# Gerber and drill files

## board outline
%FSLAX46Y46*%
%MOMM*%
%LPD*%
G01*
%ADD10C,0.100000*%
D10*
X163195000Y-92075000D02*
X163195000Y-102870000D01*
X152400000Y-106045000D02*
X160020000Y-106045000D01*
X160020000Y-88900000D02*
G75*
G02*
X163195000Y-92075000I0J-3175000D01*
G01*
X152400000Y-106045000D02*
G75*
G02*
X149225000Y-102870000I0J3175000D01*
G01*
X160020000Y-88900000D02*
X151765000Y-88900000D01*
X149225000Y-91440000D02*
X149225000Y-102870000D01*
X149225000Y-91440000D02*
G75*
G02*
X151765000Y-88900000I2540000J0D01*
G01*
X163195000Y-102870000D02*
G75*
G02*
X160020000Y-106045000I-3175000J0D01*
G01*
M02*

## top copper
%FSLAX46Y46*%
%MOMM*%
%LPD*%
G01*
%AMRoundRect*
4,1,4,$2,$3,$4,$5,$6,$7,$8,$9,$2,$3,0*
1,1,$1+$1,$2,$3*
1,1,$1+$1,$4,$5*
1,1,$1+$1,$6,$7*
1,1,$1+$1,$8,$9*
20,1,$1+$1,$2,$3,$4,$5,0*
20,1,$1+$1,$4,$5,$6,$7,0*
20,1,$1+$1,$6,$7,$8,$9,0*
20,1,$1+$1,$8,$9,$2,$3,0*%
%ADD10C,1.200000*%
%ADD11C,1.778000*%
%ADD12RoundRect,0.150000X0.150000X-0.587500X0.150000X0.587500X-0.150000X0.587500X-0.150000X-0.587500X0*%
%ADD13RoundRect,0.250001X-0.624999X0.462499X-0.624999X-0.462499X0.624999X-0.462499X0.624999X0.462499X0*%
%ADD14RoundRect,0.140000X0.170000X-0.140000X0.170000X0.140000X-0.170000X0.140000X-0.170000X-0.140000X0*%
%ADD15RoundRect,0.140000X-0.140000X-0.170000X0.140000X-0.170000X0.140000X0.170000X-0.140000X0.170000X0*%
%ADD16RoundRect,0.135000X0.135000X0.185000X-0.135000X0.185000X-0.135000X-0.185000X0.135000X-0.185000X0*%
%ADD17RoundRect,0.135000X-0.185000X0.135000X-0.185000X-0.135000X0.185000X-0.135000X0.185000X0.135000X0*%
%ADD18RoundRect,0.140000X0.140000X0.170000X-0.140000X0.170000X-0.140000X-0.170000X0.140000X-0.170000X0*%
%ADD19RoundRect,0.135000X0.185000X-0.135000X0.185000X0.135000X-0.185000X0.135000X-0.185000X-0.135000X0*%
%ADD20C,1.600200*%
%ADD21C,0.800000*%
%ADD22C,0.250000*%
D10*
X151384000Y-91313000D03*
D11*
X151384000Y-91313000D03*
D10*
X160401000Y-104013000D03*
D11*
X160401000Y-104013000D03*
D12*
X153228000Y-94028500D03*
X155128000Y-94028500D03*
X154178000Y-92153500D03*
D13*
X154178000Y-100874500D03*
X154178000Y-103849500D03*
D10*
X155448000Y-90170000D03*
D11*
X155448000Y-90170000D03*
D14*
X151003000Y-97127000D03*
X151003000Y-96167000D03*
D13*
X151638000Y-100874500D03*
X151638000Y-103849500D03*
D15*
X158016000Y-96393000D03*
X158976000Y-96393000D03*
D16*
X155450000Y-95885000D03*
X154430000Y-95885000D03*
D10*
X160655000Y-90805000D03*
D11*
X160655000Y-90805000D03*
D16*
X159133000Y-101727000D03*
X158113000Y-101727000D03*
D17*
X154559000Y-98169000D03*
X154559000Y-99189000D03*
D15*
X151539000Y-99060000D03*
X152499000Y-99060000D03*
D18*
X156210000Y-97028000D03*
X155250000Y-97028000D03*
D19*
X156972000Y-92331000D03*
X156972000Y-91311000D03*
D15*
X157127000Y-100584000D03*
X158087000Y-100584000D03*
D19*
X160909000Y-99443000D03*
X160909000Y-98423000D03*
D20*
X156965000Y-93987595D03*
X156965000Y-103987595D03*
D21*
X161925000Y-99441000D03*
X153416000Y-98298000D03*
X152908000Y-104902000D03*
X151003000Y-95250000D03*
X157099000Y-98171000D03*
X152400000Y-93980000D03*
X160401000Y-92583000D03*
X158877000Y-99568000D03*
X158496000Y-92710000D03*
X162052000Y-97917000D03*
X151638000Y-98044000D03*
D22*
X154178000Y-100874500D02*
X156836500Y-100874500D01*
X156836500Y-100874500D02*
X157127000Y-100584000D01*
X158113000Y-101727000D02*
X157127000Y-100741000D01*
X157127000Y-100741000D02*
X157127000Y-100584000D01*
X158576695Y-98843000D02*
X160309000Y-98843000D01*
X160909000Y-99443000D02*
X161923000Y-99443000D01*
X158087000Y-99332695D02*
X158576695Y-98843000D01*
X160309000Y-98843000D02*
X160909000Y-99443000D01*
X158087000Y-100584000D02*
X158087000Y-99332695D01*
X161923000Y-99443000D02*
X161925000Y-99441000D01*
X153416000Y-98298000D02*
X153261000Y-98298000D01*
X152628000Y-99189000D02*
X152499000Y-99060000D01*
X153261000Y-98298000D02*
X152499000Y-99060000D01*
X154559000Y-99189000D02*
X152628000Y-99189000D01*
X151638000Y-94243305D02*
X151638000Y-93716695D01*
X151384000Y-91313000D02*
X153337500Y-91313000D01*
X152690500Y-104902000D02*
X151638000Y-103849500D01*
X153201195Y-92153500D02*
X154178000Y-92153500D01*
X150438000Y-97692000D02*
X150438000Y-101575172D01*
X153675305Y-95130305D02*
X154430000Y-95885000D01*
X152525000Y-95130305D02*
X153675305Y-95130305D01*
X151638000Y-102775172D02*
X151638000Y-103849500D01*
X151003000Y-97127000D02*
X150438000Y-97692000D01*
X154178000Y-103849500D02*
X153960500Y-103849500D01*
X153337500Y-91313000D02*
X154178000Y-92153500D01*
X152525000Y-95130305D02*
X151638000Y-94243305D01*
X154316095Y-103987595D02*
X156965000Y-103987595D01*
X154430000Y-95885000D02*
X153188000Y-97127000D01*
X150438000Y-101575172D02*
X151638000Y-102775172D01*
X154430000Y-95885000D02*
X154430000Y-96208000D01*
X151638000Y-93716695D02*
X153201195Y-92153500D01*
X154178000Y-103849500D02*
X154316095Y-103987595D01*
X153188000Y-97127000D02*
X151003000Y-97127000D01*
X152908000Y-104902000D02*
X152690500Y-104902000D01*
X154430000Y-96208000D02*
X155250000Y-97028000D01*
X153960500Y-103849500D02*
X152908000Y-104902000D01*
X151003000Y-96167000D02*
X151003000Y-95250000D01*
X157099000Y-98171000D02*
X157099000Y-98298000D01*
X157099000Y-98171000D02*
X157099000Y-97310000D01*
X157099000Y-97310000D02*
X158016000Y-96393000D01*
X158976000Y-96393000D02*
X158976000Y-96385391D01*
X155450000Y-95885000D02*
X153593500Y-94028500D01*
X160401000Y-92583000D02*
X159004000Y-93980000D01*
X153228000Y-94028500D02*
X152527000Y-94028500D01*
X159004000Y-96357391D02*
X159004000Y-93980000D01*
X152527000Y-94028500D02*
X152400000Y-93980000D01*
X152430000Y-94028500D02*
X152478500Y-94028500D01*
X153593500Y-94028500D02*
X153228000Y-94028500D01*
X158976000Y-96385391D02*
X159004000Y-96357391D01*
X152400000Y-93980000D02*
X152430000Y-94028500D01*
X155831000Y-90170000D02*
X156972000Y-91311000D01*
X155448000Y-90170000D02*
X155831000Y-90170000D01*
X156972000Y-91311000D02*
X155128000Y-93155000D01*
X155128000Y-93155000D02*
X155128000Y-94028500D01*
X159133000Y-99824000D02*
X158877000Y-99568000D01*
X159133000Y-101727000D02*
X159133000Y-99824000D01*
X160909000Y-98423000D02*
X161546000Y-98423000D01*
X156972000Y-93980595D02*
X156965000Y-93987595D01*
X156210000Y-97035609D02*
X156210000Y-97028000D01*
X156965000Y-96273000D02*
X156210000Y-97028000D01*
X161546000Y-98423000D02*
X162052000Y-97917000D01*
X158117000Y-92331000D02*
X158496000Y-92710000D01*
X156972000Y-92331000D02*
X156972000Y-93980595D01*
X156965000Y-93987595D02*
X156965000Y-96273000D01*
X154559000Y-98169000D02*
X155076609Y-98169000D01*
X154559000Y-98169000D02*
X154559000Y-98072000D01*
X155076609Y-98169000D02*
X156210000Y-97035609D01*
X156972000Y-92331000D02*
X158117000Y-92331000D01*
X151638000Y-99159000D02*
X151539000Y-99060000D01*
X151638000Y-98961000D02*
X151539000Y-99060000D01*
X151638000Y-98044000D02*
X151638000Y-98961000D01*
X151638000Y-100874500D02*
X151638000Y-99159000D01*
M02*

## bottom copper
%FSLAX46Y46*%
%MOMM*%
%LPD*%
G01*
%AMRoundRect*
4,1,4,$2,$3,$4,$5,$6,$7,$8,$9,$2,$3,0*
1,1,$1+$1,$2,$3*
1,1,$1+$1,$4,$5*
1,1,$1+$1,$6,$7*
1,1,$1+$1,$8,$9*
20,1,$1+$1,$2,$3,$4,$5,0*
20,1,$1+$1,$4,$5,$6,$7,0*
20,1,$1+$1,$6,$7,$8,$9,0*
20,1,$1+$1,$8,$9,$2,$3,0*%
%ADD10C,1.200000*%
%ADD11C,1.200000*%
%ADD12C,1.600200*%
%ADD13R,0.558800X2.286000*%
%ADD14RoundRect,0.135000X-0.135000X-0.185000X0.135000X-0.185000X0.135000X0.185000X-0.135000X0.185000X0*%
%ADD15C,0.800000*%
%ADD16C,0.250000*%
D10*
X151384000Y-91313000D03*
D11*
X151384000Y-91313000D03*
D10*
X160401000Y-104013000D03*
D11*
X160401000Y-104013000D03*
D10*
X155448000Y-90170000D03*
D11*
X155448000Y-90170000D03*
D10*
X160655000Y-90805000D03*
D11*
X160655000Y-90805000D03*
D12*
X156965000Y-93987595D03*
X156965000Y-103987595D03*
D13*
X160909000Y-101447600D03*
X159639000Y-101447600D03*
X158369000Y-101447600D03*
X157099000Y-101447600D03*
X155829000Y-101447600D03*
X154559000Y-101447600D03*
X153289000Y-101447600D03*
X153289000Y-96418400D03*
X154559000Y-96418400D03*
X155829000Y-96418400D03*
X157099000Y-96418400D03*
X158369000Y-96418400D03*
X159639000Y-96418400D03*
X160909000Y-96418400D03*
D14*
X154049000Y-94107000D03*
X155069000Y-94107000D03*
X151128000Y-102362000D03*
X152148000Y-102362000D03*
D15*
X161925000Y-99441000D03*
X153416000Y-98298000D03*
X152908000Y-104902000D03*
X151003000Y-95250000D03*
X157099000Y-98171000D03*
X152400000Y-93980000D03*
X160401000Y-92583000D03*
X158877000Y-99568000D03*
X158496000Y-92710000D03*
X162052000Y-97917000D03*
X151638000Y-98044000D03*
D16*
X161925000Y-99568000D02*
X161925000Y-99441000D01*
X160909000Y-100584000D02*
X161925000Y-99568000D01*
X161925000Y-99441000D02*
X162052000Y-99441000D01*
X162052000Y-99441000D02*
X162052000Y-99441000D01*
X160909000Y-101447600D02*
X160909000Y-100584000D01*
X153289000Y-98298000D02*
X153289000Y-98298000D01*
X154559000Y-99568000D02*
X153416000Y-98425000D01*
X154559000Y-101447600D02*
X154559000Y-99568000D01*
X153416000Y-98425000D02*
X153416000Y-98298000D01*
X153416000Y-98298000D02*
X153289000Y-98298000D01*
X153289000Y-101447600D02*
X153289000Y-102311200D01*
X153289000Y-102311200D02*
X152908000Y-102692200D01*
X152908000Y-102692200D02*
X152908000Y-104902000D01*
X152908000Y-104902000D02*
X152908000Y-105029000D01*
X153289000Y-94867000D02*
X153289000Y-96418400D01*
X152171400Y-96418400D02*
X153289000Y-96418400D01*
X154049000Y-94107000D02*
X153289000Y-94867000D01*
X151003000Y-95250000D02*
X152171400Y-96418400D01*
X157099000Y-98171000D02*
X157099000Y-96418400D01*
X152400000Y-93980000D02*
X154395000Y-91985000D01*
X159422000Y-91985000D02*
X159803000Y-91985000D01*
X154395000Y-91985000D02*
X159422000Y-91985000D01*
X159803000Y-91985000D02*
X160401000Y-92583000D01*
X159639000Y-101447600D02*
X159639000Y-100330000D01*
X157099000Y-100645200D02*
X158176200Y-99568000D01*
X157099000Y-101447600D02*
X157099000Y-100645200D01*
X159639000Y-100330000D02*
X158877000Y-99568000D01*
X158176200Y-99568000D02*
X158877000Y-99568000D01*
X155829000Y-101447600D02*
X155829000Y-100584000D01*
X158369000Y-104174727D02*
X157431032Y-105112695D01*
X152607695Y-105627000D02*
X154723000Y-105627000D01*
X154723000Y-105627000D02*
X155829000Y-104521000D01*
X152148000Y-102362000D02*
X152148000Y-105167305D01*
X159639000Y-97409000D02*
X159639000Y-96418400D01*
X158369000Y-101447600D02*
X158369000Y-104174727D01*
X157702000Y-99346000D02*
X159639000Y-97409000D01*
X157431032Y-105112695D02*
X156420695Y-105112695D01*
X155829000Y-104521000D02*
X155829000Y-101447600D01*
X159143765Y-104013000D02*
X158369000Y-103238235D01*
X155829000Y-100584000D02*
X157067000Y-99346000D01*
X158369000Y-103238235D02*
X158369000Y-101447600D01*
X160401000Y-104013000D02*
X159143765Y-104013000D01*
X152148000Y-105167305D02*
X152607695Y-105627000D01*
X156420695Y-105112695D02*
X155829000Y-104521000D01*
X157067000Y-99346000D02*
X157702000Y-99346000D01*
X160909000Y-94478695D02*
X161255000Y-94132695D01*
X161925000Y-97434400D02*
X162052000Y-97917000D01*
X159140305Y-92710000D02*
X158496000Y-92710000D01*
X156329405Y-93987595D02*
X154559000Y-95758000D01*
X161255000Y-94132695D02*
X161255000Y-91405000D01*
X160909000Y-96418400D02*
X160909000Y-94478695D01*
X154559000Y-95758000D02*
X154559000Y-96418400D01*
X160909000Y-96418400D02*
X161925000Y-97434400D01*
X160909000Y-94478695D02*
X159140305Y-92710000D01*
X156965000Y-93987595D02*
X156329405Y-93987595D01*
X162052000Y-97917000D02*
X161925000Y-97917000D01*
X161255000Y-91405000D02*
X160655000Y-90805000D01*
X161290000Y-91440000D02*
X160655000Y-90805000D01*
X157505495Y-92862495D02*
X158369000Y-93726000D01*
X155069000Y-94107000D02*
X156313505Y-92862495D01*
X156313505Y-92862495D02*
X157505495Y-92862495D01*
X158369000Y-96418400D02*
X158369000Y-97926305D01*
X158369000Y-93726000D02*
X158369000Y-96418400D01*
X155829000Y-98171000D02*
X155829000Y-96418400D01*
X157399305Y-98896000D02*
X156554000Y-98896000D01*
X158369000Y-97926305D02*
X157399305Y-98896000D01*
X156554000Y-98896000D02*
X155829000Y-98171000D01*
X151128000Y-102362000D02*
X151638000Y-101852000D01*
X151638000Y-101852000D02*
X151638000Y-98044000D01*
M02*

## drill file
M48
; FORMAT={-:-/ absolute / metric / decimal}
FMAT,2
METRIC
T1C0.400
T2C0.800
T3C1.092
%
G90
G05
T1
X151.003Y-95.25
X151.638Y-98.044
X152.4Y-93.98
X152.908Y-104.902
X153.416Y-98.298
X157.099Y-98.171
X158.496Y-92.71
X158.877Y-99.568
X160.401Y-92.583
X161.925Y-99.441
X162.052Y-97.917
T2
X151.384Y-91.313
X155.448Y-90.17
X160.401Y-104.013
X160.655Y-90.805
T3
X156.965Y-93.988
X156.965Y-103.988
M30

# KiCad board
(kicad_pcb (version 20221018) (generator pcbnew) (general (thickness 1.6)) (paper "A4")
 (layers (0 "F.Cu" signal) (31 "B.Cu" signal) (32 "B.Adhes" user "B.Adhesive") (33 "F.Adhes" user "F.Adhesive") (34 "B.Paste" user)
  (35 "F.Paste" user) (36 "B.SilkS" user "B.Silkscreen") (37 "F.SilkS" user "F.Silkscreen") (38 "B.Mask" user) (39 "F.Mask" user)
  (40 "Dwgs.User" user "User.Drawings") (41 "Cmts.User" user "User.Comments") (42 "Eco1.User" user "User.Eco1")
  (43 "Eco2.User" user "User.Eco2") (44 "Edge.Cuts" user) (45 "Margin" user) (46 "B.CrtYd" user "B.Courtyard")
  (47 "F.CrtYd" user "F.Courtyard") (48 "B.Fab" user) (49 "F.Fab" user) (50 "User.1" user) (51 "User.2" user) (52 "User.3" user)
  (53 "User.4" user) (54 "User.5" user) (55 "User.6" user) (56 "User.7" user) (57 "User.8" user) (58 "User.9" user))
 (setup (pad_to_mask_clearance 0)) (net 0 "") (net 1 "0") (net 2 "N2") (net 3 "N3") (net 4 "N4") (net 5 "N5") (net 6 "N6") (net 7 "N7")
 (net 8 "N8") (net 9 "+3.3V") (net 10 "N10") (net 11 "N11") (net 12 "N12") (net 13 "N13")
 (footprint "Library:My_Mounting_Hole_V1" (layer "F.Cu") (at 151.384 91.313)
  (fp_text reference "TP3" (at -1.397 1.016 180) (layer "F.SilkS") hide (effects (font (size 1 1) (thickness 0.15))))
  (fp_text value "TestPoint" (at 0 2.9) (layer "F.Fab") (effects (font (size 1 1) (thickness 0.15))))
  (pad "1" thru_hole circle (at 0 0) (size 1.2 1.2) (drill 0.8) (layers "*.Cu" "*.Mask") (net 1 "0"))
  (pad "1" connect circle (at 0 0) (size 1.2 1.2) (layers "B.Cu" "B.Mask") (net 1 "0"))
  (pad "1" connect circle (at 0 0) (size 1.778 1.778) (layers "F.Cu" "F.Mask") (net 1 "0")))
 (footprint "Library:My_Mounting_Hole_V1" (layer "F.Cu") (at 160.401 104.013)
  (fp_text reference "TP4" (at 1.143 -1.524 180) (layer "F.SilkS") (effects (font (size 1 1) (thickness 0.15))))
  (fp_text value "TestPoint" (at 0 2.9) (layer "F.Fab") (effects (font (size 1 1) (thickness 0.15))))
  (pad "1" thru_hole circle (at 0 0) (size 1.2 1.2) (drill 0.8) (layers "*.Cu" "*.Mask") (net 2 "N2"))
  (pad "1" connect circle (at 0 0) (size 1.2 1.2) (layers "B.Cu" "B.Mask") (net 2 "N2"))
  (pad "1" connect circle (at 0 0) (size 1.778 1.778) (layers "F.Cu" "F.Mask") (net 2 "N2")))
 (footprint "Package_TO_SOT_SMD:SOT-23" (layer "F.Cu") (at 154.178 93.091 90)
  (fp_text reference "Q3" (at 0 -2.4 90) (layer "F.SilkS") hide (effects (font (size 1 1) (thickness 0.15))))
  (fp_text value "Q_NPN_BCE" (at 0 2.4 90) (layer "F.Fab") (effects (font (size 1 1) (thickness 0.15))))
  (pad "1" smd roundrect (at -0.9375 -0.95 90) (size 1.475 0.6) (layers "F.Cu" "F.Paste" "F.Mask") (roundrect_rratio 0.25) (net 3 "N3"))
  (pad "2" smd roundrect (at -0.9375 0.95 90) (size 1.475 0.6) (layers "F.Cu" "F.Paste" "F.Mask") (roundrect_rratio 0.25) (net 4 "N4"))
  (pad "3" smd roundrect (at 0.9375 0 90) (size 1.475 0.6) (layers "F.Cu" "F.Paste" "F.Mask") (roundrect_rratio 0.25) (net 1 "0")))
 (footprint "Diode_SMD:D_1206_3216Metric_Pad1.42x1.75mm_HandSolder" (layer "F.Cu") (at 154.178 102.362 -90)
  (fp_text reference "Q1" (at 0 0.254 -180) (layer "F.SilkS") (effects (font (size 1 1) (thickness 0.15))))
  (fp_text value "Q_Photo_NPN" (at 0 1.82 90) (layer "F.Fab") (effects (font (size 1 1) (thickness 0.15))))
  (pad "1" smd roundrect (at -1.4875 0 270) (size 1.425 1.75) (layers "F.Cu" "F.Paste" "F.Mask") (roundrect_rratio 0.1754392982)
   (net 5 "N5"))
  (pad "2" smd roundrect (at 1.4875 0 270) (size 1.425 1.75) (layers "F.Cu" "F.Paste" "F.Mask") (roundrect_rratio 0.1754392982) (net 1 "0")))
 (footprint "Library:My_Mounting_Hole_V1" (layer "F.Cu") (at 155.448 90.17)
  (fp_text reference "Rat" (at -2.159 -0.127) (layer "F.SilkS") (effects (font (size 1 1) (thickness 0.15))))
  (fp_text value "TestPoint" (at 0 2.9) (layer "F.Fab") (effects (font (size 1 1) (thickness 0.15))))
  (pad "1" thru_hole circle (at 0 0) (size 1.2 1.2) (drill 0.8) (layers "*.Cu" "*.Mask") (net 4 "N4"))
  (pad "1" connect circle (at 0 0) (size 1.2 1.2) (layers "B.Cu" "B.Mask") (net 4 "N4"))
  (pad "1" connect circle (at 0 0) (size 1.778 1.778) (layers "F.Cu" "F.Mask") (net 4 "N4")))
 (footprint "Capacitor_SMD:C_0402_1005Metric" (layer "F.Cu") (at 151.003 96.647 90)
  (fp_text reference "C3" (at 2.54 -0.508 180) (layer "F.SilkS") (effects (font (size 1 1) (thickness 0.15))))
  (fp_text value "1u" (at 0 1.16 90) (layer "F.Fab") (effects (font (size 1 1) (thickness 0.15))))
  (pad "1" smd roundrect (at -0.48 0 90) (size 0.56 0.62) (layers "F.Cu" "F.Paste" "F.Mask") (roundrect_rratio 0.25) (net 1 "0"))
  (pad "2" smd roundrect (at 0.48 0 90) (size 0.56 0.62) (layers "F.Cu" "F.Paste" "F.Mask") (roundrect_rratio 0.25) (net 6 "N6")))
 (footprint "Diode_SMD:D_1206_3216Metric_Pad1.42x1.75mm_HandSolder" (layer "F.Cu") (at 151.638 102.362 -90)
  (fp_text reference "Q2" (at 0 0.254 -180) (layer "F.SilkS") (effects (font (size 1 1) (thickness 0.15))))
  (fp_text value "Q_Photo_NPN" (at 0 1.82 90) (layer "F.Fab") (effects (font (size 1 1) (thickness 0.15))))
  (pad "1" smd roundrect (at -1.4875 0 270) (size 1.425 1.75) (layers "F.Cu" "F.Paste" "F.Mask") (roundrect_rratio 0.1754392982)
   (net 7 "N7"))
  (pad "2" smd roundrect (at 1.4875 0 270) (size 1.425 1.75) (layers "F.Cu" "F.Paste" "F.Mask") (roundrect_rratio 0.1754392982) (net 1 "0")))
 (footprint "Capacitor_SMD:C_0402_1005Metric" (layer "F.Cu") (at 158.496 96.393)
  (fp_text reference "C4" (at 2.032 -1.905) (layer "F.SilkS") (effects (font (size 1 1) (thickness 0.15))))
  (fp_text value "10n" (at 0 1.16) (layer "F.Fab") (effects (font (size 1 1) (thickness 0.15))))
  (pad "1" smd roundrect (at -0.48 0) (size 0.56 0.62) (layers "F.Cu" "F.Paste" "F.Mask") (roundrect_rratio 0.25) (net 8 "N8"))
  (pad "2" smd roundrect (at 0.48 0) (size 0.56 0.62) (layers "F.Cu" "F.Paste" "F.Mask") (roundrect_rratio 0.25) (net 3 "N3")))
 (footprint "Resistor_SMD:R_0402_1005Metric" (layer "F.Cu") (at 154.94 95.885 180)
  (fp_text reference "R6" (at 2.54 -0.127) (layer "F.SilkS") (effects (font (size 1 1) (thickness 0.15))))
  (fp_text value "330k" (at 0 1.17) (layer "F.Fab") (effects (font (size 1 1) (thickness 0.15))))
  (pad "1" smd roundrect (at -0.51 0 180) (size 0.54 0.64) (layers "F.Cu" "F.Paste" "F.Mask") (roundrect_rratio 0.25) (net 3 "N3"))
  (pad "2" smd roundrect (at 0.51 0 180) (size 0.54 0.64) (layers "F.Cu" "F.Paste" "F.Mask") (roundrect_rratio 0.25) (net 1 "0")))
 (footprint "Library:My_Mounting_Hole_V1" (layer "F.Cu") (at 160.655 90.805)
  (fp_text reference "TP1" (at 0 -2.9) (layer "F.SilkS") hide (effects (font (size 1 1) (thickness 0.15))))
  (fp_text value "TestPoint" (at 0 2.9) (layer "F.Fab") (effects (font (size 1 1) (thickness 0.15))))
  (pad "1" thru_hole circle (at 0 0) (size 1.2 1.2) (drill 0.8) (layers "*.Cu" "*.Mask") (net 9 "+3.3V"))
  (pad "1" connect circle (at 0 0) (size 1.2 1.2) (layers "B.Cu" "B.Mask") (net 9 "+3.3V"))
  (pad "1" connect circle (at 0 0) (size 1.778 1.778) (layers "F.Cu" "F.Mask") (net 9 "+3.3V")))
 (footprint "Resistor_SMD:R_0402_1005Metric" (layer "F.Cu") (at 158.623 101.727 180)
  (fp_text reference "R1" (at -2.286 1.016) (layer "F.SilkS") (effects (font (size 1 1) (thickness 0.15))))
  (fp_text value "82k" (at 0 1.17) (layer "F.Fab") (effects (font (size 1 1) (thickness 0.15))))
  (pad "1" smd roundrect (at -0.51 0 180) (size 0.54 0.64) (layers "F.Cu" "F.Paste" "F.Mask") (roundrect_rratio 0.25) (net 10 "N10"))
  (pad "2" smd roundrect (at 0.51 0 180) (size 0.54 0.64) (layers "F.Cu" "F.Paste" "F.Mask") (roundrect_rratio 0.25) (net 5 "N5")))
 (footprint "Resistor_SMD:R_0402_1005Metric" (layer "F.Cu") (at 154.559 98.679 -90)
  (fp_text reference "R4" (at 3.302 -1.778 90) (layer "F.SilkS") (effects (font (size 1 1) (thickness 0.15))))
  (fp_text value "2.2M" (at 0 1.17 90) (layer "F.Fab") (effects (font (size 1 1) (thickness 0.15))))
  (pad "1" smd roundrect (at -0.51 0 270) (size 0.54 0.64) (layers "F.Cu" "F.Paste" "F.Mask") (roundrect_rratio 0.25) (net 9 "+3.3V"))
  (pad "2" smd roundrect (at 0.51 0 270) (size 0.54 0.64) (layers "F.Cu" "F.Paste" "F.Mask") (roundrect_rratio 0.25) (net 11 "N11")))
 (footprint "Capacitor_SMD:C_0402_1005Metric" (layer "F.Cu") (at 152.019 99.06)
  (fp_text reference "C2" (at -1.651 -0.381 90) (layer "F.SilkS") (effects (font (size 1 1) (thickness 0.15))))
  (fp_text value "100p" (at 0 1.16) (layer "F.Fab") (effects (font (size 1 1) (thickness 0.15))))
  (pad "1" smd roundrect (at -0.48 0) (size 0.56 0.62) (layers "F.Cu" "F.Paste" "F.Mask") (roundrect_rratio 0.25) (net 7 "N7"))
  (pad "2" smd roundrect (at 0.48 0) (size 0.56 0.62) (layers "F.Cu" "F.Paste" "F.Mask") (roundrect_rratio 0.25) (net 11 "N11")))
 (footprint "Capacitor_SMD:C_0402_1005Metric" (layer "F.Cu") (at 155.73 97.028 180)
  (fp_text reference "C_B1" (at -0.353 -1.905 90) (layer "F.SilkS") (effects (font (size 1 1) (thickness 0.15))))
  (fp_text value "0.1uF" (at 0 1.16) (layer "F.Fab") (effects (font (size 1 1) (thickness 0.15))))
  (pad "1" smd roundrect (at -0.48 0 180) (size 0.56 0.62) (layers "F.Cu" "F.Paste" "F.Mask") (roundrect_rratio 0.25) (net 9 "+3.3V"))
  (pad "2" smd roundrect (at 0.48 0 180) (size 0.56 0.62) (layers "F.Cu" "F.Paste" "F.Mask") (roundrect_rratio 0.25) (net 1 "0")))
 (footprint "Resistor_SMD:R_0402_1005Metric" (layer "F.Cu") (at 156.972 91.821 90)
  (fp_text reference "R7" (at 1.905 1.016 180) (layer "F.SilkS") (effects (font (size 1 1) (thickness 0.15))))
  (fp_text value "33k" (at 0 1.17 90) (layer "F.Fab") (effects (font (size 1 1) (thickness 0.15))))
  (pad "1" smd roundrect (at -0.51 0 90) (size 0.54 0.64) (layers "F.Cu" "F.Paste" "F.Mask") (roundrect_rratio 0.25) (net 9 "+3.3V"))
  (pad "2" smd roundrect (at 0.51 0 90) (size 0.54 0.64) (layers "F.Cu" "F.Paste" "F.Mask") (roundrect_rratio 0.25) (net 4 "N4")))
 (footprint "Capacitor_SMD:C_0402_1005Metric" (layer "F.Cu") (at 157.607 100.584)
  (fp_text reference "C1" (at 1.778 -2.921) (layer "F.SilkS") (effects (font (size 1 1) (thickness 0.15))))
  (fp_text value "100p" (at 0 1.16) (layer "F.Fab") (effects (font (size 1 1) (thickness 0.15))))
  (pad "1" smd roundrect (at -0.48 0) (size 0.56 0.62) (layers "F.Cu" "F.Paste" "F.Mask") (roundrect_rratio 0.25) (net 5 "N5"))
  (pad "2" smd roundrect (at 0.48 0) (size 0.56 0.62) (layers "F.Cu" "F.Paste" "F.Mask") (roundrect_rratio 0.25) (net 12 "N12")))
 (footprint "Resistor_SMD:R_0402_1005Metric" (layer "F.Cu") (at 160.909 98.933 90)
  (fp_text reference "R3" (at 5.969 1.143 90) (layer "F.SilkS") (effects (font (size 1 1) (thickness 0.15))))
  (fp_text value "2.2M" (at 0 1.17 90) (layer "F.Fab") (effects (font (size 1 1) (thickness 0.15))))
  (pad "1" smd roundrect (at -0.51 0 90) (size 0.54 0.64) (layers "F.Cu" "F.Paste" "F.Mask") (roundrect_rratio 0.25) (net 12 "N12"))
  (pad "2" smd roundrect (at 0.51 0 90) (size 0.54 0.64) (layers "F.Cu" "F.Paste" "F.Mask") (roundrect_rratio 0.25) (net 9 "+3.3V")))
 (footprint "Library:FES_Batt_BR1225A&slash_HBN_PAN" (layer "B.Cu") (at 156.965 93.987595 180)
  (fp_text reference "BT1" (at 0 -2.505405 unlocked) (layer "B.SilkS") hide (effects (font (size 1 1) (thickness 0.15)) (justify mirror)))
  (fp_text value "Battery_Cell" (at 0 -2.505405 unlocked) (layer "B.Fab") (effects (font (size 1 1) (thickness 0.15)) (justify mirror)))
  (pad "1" thru_hole circle (at 0 0 180) (size 1.6002 1.6002) (drill 1.0922) (layers "*.Cu" "*.Mask") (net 9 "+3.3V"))
  (pad "2" thru_hole circle (at 0 -10 180) (size 1.6002 1.6002) (drill 1.0922) (layers "*.Cu" "*.Mask") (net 1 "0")))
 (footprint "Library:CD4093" (layer "B.Cu") (at 157.099 98.933 90)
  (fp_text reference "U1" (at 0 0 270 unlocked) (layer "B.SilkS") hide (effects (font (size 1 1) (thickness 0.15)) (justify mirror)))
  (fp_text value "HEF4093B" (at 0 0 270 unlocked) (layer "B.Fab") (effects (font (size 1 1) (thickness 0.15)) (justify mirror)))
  (pad "1" smd rect (at -2.5146 3.81 90) (size 2.286 0.5588) (layers "B.Cu" "B.Paste" "B.Mask") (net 12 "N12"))
  (pad "2" smd rect (at -2.5146 2.54 90) (size 2.286 0.5588) (layers "B.Cu" "B.Paste" "B.Mask") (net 10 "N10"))
  (pad "3" smd rect (at -2.5146 1.27 90) (size 2.286 0.5588) (layers "B.Cu" "B.Paste" "B.Mask") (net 2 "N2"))
  (pad "4" smd rect (at -2.5146 0 90) (size 2.286 0.5588) (layers "B.Cu" "B.Paste" "B.Mask") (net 10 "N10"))
  (pad "5" smd rect (at -2.5146 -1.27 90) (size 2.286 0.5588) (layers "B.Cu" "B.Paste" "B.Mask") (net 2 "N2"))
  (pad "6" smd rect (at -2.5146 -2.54 90) (size 2.286 0.5588) (layers "B.Cu" "B.Paste" "B.Mask") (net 11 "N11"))
  (pad "7" smd rect (at -2.5146 -3.81 90) (size 2.286 0.5588) (layers "B.Cu" "B.Paste" "B.Mask") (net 1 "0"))
  (pad "8" smd rect (at 2.5146 -3.81 90) (size 2.286 0.5588) (layers "B.Cu" "B.Paste" "B.Mask") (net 6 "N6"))
  (pad "9" smd rect (at 2.5146 -2.54 90) (size 2.286 0.5588) (layers "B.Cu" "B.Paste" "B.Mask") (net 9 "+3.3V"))
  (pad "10" smd rect (at 2.5146 -1.27 90) (size 2.286 0.5588) (layers "B.Cu" "B.Paste" "B.Mask") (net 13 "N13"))
  (pad "11" smd rect (at 2.5146 0 90) (size 2.286 0.5588) (layers "B.Cu" "B.Paste" "B.Mask") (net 8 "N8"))
  (pad "12" smd rect (at 2.5146 1.27 90) (size 2.286 0.5588) (layers "B.Cu" "B.Paste" "B.Mask") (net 13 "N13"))
  (pad "13" smd rect (at 2.5146 2.54 90) (size 2.286 0.5588) (layers "B.Cu" "B.Paste" "B.Mask") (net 2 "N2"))
  (pad "14" smd rect (at 2.5146 3.81 90) (size 2.286 0.5588) (layers "B.Cu" "B.Paste" "B.Mask") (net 9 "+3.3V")))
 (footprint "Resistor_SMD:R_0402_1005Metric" (layer "B.Cu") (at 154.559 94.107)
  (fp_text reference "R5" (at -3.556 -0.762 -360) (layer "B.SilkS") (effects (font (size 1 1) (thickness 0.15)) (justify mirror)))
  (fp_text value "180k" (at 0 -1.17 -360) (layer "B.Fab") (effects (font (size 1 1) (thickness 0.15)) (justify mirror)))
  (pad "1" smd roundrect (at -0.51 0) (size 0.54 0.64) (layers "B.Cu" "B.Paste" "B.Mask") (roundrect_rratio 0.25) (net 6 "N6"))
  (pad "2" smd roundrect (at 0.51 0) (size 0.54 0.64) (layers "B.Cu" "B.Paste" "B.Mask") (roundrect_rratio 0.25) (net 13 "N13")))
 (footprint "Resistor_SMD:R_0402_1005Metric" (layer "B.Cu") (at 151.638 102.362)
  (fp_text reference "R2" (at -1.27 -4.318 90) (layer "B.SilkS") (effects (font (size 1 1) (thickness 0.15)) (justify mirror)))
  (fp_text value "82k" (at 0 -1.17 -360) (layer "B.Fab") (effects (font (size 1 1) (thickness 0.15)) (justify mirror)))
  (pad "1" smd roundrect (at -0.51 0) (size 0.54 0.64) (layers "B.Cu" "B.Paste" "B.Mask") (roundrect_rratio 0.25) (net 7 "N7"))
  (pad "2" smd roundrect (at 0.51 0) (size 0.54 0.64) (layers "B.Cu" "B.Paste" "B.Mask") (roundrect_rratio 0.25) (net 2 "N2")))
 (gr_line (start 163.195 92.075) (end 163.195 102.87) (stroke (width 0.1) (type default)) (layer "Edge.Cuts"))
 (gr_line (start 152.4 106.045) (end 160.02 106.045) (stroke (width 0.1) (type default)) (layer "Edge.Cuts"))
 (gr_arc (start 160.02 88.9) (mid 162.265064 89.829936) (end 163.195 92.075) (stroke (width 0.1) (type default)) (layer "Edge.Cuts"))
 (gr_arc (start 152.4 106.045) (mid 150.154936 105.115064) (end 149.225 102.87) (stroke (width 0.1) (type default)) (layer "Edge.Cuts"))
 (gr_line (start 160.02 88.9) (end 151.765 88.9) (stroke (width 0.1) (type default)) (layer "Edge.Cuts"))
 (gr_line (start 149.225 91.44) (end 149.225 102.87) (stroke (width 0.1) (type default)) (layer "Edge.Cuts"))
 (gr_arc (start 149.225 91.44) (mid 149.968949 89.643949) (end 151.765 88.9) (stroke (width 0.1) (type default)) (layer "Edge.Cuts"))
 (gr_arc (start 163.195 102.87) (mid 162.265064 105.115064) (end 160.02 106.045) (stroke (width 0.1) (type default)) (layer "Edge.Cuts"))
 (segment (start 154.178 100.8745) (end 156.8365 100.8745) (width 0.25) (layer "F.Cu") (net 5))
 (segment (start 156.8365 100.8745) (end 157.127 100.584) (width 0.25) (layer "F.Cu") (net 5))
 (segment (start 158.113 101.727) (end 157.127 100.741) (width 0.25) (layer "F.Cu") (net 5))
 (segment (start 157.127 100.741) (end 157.127 100.584) (width 0.25) (layer "F.Cu") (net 5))
 (segment (start 158.576695 98.843) (end 160.309 98.843) (width 0.25) (layer "F.Cu") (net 12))
 (segment (start 160.909 99.443) (end 161.923 99.443) (width 0.25) (layer "F.Cu") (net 12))
 (segment (start 158.087 99.332695) (end 158.576695 98.843) (width 0.25) (layer "F.Cu") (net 12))
 (segment (start 160.309 98.843) (end 160.909 99.443) (width 0.25) (layer "F.Cu") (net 12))
 (segment (start 158.087 100.584) (end 158.087 99.332695) (width 0.25) (layer "F.Cu") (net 12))
 (segment (start 161.923 99.443) (end 161.925 99.441) (width 0.25) (layer "F.Cu") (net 12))
 (via (at 161.925 99.441) (size 0.8) (drill 0.4) (layers "F.Cu" "B.Cu") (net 12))
 (segment (start 161.925 99.568) (end 161.925 99.441) (width 0.25) (layer "B.Cu") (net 12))
 (segment (start 160.909 100.584) (end 161.925 99.568) (width 0.25) (layer "B.Cu") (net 12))
 (segment (start 161.925 99.441) (end 162.052 99.441) (width 0.25) (layer "B.Cu") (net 12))
 (segment (start 162.052 99.441) (end 162.052 99.441) (width 0.25) (layer "B.Cu") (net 12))
 (segment (start 160.909 101.4476) (end 160.909 100.584) (width 0.25) (layer "B.Cu") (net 12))
 (segment (start 153.416 98.298) (end 153.261 98.298) (width 0.25) (layer "F.Cu") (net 11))
 (segment (start 152.628 99.189) (end 152.499 99.06) (width 0.25) (layer "F.Cu") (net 11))
 (segment (start 153.261 98.298) (end 152.499 99.06) (width 0.25) (layer "F.Cu") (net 11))
 (segment (start 154.559 99.189) (end 152.628 99.189) (width 0.25) (layer "F.Cu") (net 11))
 (via (at 153.416 98.298) (size 0.8) (drill 0.4) (layers "F.Cu" "B.Cu") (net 11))
 (segment (start 153.289 98.298) (end 153.289 98.298) (width 0.25) (layer "B.Cu") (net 11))
 (segment (start 154.559 99.568) (end 153.416 98.425) (width 0.25) (layer "B.Cu") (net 11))
 (segment (start 154.559 101.4476) (end 154.559 99.568) (width 0.25) (layer "B.Cu") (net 11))
 (segment (start 153.416 98.425) (end 153.416 98.298) (width 0.25) (layer "B.Cu") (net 11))
 (segment (start 153.416 98.298) (end 153.289 98.298) (width 0.25) (layer "B.Cu") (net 11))
 (segment (start 151.638 94.243305) (end 151.638 93.716695) (width 0.25) (layer "F.Cu") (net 1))
 (segment (start 151.384 91.313) (end 153.3375 91.313) (width 0.25) (layer "F.Cu") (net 1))
 (segment (start 152.6905 104.902) (end 151.638 103.8495) (width 0.25) (layer "F.Cu") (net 1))
 (segment (start 153.201195 92.1535) (end 154.178 92.1535) (width 0.25) (layer "F.Cu") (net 1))
 (segment (start 150.438 97.692) (end 150.438 101.575172) (width 0.25) (layer "F.Cu") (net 1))
 (segment (start 153.675305 95.130305) (end 154.43 95.885) (width 0.25) (layer "F.Cu") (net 1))
 (segment (start 152.525 95.130305) (end 153.675305 95.130305) (width 0.25) (layer "F.Cu") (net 1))
 (segment (start 151.638 102.775172) (end 151.638 103.8495) (width 0.25) (layer "F.Cu") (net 1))
 (segment (start 151.003 97.127) (end 150.438 97.692) (width 0.25) (layer "F.Cu") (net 1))
 (segment (start 154.178 103.8495) (end 153.9605 103.8495) (width 0.25) (layer "F.Cu") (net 1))
 (segment (start 153.3375 91.313) (end 154.178 92.1535) (width 0.25) (layer "F.Cu") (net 1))
 (segment (start 152.525 95.130305) (end 151.638 94.243305) (width 0.25) (layer "F.Cu") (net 1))
 (segment (start 154.316095 103.987595) (end 156.965 103.987595) (width 0.25) (layer "F.Cu") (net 1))
 (segment (start 154.43 95.885) (end 153.188 97.127) (width 0.25) (layer "F.Cu") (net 1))
 (segment (start 150.438 101.575172) (end 151.638 102.775172) (width 0.25) (layer "F.Cu") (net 1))
 (segment (start 154.43 95.885) (end 154.43 96.208) (width 0.25) (layer "F.Cu") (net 1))
 (segment (start 151.638 93.716695) (end 153.201195 92.1535) (width 0.25) (layer "F.Cu") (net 1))
 (segment (start 154.178 103.8495) (end 154.316095 103.987595) (width 0.25) (layer "F.Cu") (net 1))
 (segment (start 153.188 97.127) (end 151.003 97.127) (width 0.25) (layer "F.Cu") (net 1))
 (segment (start 152.908 104.902) (end 152.6905 104.902) (width 0.25) (layer "F.Cu") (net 1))
 (segment (start 154.43 96.208) (end 155.25 97.028) (width 0.25) (layer "F.Cu") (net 1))
 (segment (start 153.9605 103.8495) (end 152.908 104.902) (width 0.25) (layer "F.Cu") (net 1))
 (via (at 152.908 104.902) (size 0.8) (drill 0.4) (layers "F.Cu" "B.Cu") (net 1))
 (segment (start 153.289 101.4476) (end 153.289 102.3112) (width 0.25) (layer "B.Cu") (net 1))
 (segment (start 153.289 102.3112) (end 152.908 102.6922) (width 0.25) (layer "B.Cu") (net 1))
 (segment (start 152.908 102.6922) (end 152.908 104.902) (width 0.25) (layer "B.Cu") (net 1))
 (segment (start 152.908 104.902) (end 152.908 105.029) (width 0.25) (layer "B.Cu") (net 1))
 (segment (start 151.003 96.167) (end 151.003 95.25) (width 0.25) (layer "F.Cu") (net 6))
 (via (at 151.003 95.25) (size 0.8) (drill 0.4) (layers "F.Cu" "B.Cu") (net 6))
 (segment (start 153.289 94.867) (end 153.289 96.4184) (width 0.25) (layer "B.Cu") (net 6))
 (segment (start 152.1714 96.4184) (end 153.289 96.4184) (width 0.25) (layer "B.Cu") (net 6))
 (segment (start 154.049 94.107) (end 153.289 94.867) (width 0.25) (layer "B.Cu") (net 6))
 (segment (start 151.003 95.25) (end 152.1714 96.4184) (width 0.25) (layer "B.Cu") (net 6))
 (segment (start 157.099 98.171) (end 157.099 98.298) (width 0.25) (layer "F.Cu") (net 8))
 (segment (start 157.099 98.171) (end 157.099 97.31) (width 0.25) (layer "F.Cu") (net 8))
 (segment (start 157.099 97.31) (end 158.016 96.393) (width 0.25) (layer "F.Cu") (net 8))
 (via (at 157.099 98.171) (size 0.8) (drill 0.4) (layers "F.Cu" "B.Cu") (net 8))
 (segment (start 157.099 98.171) (end 157.099 96.4184) (width 0.25) (layer "B.Cu") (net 8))
 (segment (start 158.976 96.393) (end 158.976 96.385391) (width 0.25) (layer "F.Cu") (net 3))
 (segment (start 155.45 95.885) (end 153.5935 94.0285) (width 0.25) (layer "F.Cu") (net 3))
 (segment (start 160.401 92.583) (end 159.004 93.98) (width 0.25) (layer "F.Cu") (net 3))
 (segment (start 153.228 94.0285) (end 152.527 94.0285) (width 0.25) (layer "F.Cu") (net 3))
 (segment (start 159.004 96.357391) (end 159.004 93.98) (width 0.25) (layer "F.Cu") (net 3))
 (segment (start 152.527 94.0285) (end 152.4 93.98) (width 0.25) (layer "F.Cu") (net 3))
 (segment (start 152.43 94.0285) (end 152.4785 94.0285) (width 0.25) (layer "F.Cu") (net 3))
 (segment (start 153.5935 94.0285) (end 153.228 94.0285) (width 0.25) (layer "F.Cu") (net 3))
 (segment (start 158.976 96.385391) (end 159.004 96.357391) (width 0.25) (layer "F.Cu") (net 3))
 (segment (start 152.4 93.98) (end 152.43 94.0285) (width 0.25) (layer "F.Cu") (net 3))
 (via (at 152.4 93.98) (size 0.8) (drill 0.4) (layers "F.Cu" "B.Cu") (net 3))
 (via (at 160.401 92.583) (size 0.8) (drill 0.4) (layers "F.Cu" "B.Cu") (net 3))
 (segment (start 152.4 93.98) (end 154.395 91.985) (width 0.25) (layer "B.Cu") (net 3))
 (segment (start 159.422 91.985) (end 159.803 91.985) (width 0.25) (layer "B.Cu") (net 3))
 (segment (start 154.395 91.985) (end 159.422 91.985) (width 0.25) (layer "B.Cu") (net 3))
 (segment (start 159.803 91.985) (end 160.401 92.583) (width 0.25) (layer "B.Cu") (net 3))
 (segment (start 155.831 90.17) (end 156.972 91.311) (width 0.25) (layer "F.Cu") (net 4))
 (segment (start 155.448 90.17) (end 155.831 90.17) (width 0.25) (layer "F.Cu") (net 4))
 (segment (start 156.972 91.311) (end 155.128 93.155) (width 0.25) (layer "F.Cu") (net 4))
 (segment (start 155.128 93.155) (end 155.128 94.0285) (width 0.25) (layer "F.Cu") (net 4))
 (segment (start 159.133 99.824) (end 158.877 99.568) (width 0.25) (layer "F.Cu") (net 10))
 (segment (start 159.133 101.727) (end 159.133 99.824) (width 0.25) (layer "F.Cu") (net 10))
 (via (at 158.877 99.568) (size 0.8) (drill 0.4) (layers "F.Cu" "B.Cu") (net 10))
 (segment (start 159.639 101.4476) (end 159.639 100.33) (width 0.25) (layer "B.Cu") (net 10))
 (segment (start 157.099 100.6452) (end 158.1762 99.568) (width 0.25) (layer "B.Cu") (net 10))
 (segment (start 157.099 101.4476) (end 157.099 100.6452) (width 0.25) (layer "B.Cu") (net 10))
 (segment (start 159.639 100.33) (end 158.877 99.568) (width 0.25) (layer "B.Cu") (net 10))
 (segment (start 158.1762 99.568) (end 158.877 99.568) (width 0.25) (layer "B.Cu") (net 10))
 (segment (start 155.829 101.4476) (end 155.829 100.584) (width 0.25) (layer "B.Cu") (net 2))
 (segment (start 158.369 104.174727) (end 157.431032 105.112695) (width 0.25) (layer "B.Cu") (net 2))
 (segment (start 152.607695 105.627) (end 154.723 105.627) (width 0.25) (layer "B.Cu") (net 2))
 (segment (start 154.723 105.627) (end 155.829 104.521) (width 0.25) (layer "B.Cu") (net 2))
 (segment (start 152.148 102.362) (end 152.148 105.167305) (width 0.25) (layer "B.Cu") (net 2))
 (segment (start 159.639 97.409) (end 159.639 96.4184) (width 0.25) (layer "B.Cu") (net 2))
 (segment (start 158.369 101.4476) (end 158.369 104.174727) (width 0.25) (layer "B.Cu") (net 2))
 (segment (start 157.702 99.346) (end 159.639 97.409) (width 0.25) (layer "B.Cu") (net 2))
 (segment (start 157.431032 105.112695) (end 156.420695 105.112695) (width 0.25) (layer "B.Cu") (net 2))
 (segment (start 155.829 104.521) (end 155.829 101.4476) (width 0.25) (layer "B.Cu") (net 2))
 (segment (start 159.143765 104.013) (end 158.369 103.238235) (width 0.25) (layer "B.Cu") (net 2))
 (segment (start 155.829 100.584) (end 157.067 99.346) (width 0.25) (layer "B.Cu") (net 2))
 (segment (start 158.369 103.238235) (end 158.369 101.4476) (width 0.25) (layer "B.Cu") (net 2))
 (segment (start 160.401 104.013) (end 159.143765 104.013) (width 0.25) (layer "B.Cu") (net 2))
 (segment (start 152.148 105.167305) (end 152.607695 105.627) (width 0.25) (layer "B.Cu") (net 2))
 (segment (start 156.420695 105.112695) (end 155.829 104.521) (width 0.25) (layer "B.Cu") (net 2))
 (segment (start 157.067 99.346) (end 157.702 99.346) (width 0.25) (layer "B.Cu") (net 2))
 (segment (start 160.909 98.423) (end 161.546 98.423) (width 0.25) (layer "F.Cu") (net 9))
 (segment (start 156.972 93.980595) (end 156.965 93.987595) (width 0.25) (layer "F.Cu") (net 9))
 (segment (start 156.21 97.035609) (end 156.21 97.028) (width 0.25) (layer "F.Cu") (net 9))
 (segment (start 156.965 96.273) (end 156.21 97.028) (width 0.25) (layer "F.Cu") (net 9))
 (segment (start 161.546 98.423) (end 162.052 97.917) (width 0.25) (layer "F.Cu") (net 9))
 (segment (start 158.117 92.331) (end 158.496 92.71) (width 0.25) (layer "F.Cu") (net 9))
 (segment (start 156.972 92.331) (end 156.972 93.980595) (width 0.25) (layer "F.Cu") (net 9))
 (segment (start 156.965 93.987595) (end 156.965 96.273) (width 0.25) (layer "F.Cu") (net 9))
 (segment (start 154.559 98.169) (end 155.076609 98.169) (width 0.25) (layer "F.Cu") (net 9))
 (segment (start 154.559 98.169) (end 154.559 98.072) (width 0.25) (layer "F.Cu") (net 9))
 (segment (start 155.076609 98.169) (end 156.21 97.035609) (width 0.25) (layer "F.Cu") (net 9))
 (segment (start 156.972 92.331) (end 158.117 92.331) (width 0.25) (layer "F.Cu") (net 9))
 (via (at 158.496 92.71) (size 0.8) (drill 0.4) (layers "F.Cu" "B.Cu") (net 9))
 (via (at 162.052 97.917) (size 0.8) (drill 0.4) (layers "F.Cu" "B.Cu") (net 9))
 (segment (start 160.909 94.478695) (end 161.255 94.132695) (width 0.25) (layer "B.Cu") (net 9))
 (segment (start 161.925 97.4344) (end 162.052 97.917) (width 0.25) (layer "B.Cu") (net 9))
 (segment (start 159.140305 92.71) (end 158.496 92.71) (width 0.25) (layer "B.Cu") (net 9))
 (segment (start 156.329405 93.987595) (end 154.559 95.758) (width 0.25) (layer "B.Cu") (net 9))
 (segment (start 161.255 94.132695) (end 161.255 91.405) (width 0.25) (layer "B.Cu") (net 9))
 (segment (start 160.909 96.4184) (end 160.909 94.478695) (width 0.25) (layer "B.Cu") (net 9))
 (segment (start 154.559 95.758) (end 154.559 96.4184) (width 0.25) (layer "B.Cu") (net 9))
 (segment (start 160.909 96.4184) (end 161.925 97.4344) (width 0.25) (layer "B.Cu") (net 9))
 (segment (start 160.909 94.478695) (end 159.140305 92.71) (width 0.25) (layer "B.Cu") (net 9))
 (segment (start 156.965 93.987595) (end 156.329405 93.987595) (width 0.25) (layer "B.Cu") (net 9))
 (segment (start 162.052 97.917) (end 161.925 97.917) (width 0.25) (layer "B.Cu") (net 9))
 (segment (start 161.255 91.405) (end 160.655 90.805) (width 0.25) (layer "B.Cu") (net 9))
 (segment (start 161.29 91.44) (end 160.655 90.805) (width 0.25) (layer "B.Cu") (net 9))
 (segment (start 157.505495 92.862495) (end 158.369 93.726) (width 0.25) (layer "B.Cu") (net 13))
 (segment (start 155.069 94.107) (end 156.313505 92.862495) (width 0.25) (layer "B.Cu") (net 13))
 (segment (start 156.313505 92.862495) (end 157.505495 92.862495) (width 0.25) (layer "B.Cu") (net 13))
 (segment (start 158.369 96.4184) (end 158.369 97.926305) (width 0.25) (layer "B.Cu") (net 13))
 (segment (start 158.369 93.726) (end 158.369 96.4184) (width 0.25) (layer "B.Cu") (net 13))
 (segment (start 155.829 98.171) (end 155.829 96.4184) (width 0.25) (layer "B.Cu") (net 13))
 (segment (start 157.399305 98.896) (end 156.554 98.896) (width 0.25) (layer "B.Cu") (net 13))
 (segment (start 158.369 97.926305) (end 157.399305 98.896) (width 0.25) (layer "B.Cu") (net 13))
 (segment (start 156.554 98.896) (end 155.829 98.171) (width 0.25) (layer "B.Cu") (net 13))
 (segment (start 151.638 99.159) (end 151.539 99.06) (width 0.25) (layer "F.Cu") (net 7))
 (segment (start 151.638 98.961) (end 151.539 99.06) (width 0.25) (layer "F.Cu") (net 7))
 (segment (start 151.638 98.044) (end 151.638 98.961) (width 0.25) (layer "F.Cu") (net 7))
 (segment (start 151.638 100.8745) (end 151.638 99.159) (width 0.25) (layer "F.Cu") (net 7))
 (via (at 151.638 98.044) (size 0.8) (drill 0.4) (layers "F.Cu" "B.Cu") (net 7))
 (segment (start 151.128 102.362) (end 151.638 101.852) (width 0.25) (layer "B.Cu") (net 7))
 (segment (start 151.638 101.852) (end 151.638 98.044) (width 0.25) (layer "B.Cu") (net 7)))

